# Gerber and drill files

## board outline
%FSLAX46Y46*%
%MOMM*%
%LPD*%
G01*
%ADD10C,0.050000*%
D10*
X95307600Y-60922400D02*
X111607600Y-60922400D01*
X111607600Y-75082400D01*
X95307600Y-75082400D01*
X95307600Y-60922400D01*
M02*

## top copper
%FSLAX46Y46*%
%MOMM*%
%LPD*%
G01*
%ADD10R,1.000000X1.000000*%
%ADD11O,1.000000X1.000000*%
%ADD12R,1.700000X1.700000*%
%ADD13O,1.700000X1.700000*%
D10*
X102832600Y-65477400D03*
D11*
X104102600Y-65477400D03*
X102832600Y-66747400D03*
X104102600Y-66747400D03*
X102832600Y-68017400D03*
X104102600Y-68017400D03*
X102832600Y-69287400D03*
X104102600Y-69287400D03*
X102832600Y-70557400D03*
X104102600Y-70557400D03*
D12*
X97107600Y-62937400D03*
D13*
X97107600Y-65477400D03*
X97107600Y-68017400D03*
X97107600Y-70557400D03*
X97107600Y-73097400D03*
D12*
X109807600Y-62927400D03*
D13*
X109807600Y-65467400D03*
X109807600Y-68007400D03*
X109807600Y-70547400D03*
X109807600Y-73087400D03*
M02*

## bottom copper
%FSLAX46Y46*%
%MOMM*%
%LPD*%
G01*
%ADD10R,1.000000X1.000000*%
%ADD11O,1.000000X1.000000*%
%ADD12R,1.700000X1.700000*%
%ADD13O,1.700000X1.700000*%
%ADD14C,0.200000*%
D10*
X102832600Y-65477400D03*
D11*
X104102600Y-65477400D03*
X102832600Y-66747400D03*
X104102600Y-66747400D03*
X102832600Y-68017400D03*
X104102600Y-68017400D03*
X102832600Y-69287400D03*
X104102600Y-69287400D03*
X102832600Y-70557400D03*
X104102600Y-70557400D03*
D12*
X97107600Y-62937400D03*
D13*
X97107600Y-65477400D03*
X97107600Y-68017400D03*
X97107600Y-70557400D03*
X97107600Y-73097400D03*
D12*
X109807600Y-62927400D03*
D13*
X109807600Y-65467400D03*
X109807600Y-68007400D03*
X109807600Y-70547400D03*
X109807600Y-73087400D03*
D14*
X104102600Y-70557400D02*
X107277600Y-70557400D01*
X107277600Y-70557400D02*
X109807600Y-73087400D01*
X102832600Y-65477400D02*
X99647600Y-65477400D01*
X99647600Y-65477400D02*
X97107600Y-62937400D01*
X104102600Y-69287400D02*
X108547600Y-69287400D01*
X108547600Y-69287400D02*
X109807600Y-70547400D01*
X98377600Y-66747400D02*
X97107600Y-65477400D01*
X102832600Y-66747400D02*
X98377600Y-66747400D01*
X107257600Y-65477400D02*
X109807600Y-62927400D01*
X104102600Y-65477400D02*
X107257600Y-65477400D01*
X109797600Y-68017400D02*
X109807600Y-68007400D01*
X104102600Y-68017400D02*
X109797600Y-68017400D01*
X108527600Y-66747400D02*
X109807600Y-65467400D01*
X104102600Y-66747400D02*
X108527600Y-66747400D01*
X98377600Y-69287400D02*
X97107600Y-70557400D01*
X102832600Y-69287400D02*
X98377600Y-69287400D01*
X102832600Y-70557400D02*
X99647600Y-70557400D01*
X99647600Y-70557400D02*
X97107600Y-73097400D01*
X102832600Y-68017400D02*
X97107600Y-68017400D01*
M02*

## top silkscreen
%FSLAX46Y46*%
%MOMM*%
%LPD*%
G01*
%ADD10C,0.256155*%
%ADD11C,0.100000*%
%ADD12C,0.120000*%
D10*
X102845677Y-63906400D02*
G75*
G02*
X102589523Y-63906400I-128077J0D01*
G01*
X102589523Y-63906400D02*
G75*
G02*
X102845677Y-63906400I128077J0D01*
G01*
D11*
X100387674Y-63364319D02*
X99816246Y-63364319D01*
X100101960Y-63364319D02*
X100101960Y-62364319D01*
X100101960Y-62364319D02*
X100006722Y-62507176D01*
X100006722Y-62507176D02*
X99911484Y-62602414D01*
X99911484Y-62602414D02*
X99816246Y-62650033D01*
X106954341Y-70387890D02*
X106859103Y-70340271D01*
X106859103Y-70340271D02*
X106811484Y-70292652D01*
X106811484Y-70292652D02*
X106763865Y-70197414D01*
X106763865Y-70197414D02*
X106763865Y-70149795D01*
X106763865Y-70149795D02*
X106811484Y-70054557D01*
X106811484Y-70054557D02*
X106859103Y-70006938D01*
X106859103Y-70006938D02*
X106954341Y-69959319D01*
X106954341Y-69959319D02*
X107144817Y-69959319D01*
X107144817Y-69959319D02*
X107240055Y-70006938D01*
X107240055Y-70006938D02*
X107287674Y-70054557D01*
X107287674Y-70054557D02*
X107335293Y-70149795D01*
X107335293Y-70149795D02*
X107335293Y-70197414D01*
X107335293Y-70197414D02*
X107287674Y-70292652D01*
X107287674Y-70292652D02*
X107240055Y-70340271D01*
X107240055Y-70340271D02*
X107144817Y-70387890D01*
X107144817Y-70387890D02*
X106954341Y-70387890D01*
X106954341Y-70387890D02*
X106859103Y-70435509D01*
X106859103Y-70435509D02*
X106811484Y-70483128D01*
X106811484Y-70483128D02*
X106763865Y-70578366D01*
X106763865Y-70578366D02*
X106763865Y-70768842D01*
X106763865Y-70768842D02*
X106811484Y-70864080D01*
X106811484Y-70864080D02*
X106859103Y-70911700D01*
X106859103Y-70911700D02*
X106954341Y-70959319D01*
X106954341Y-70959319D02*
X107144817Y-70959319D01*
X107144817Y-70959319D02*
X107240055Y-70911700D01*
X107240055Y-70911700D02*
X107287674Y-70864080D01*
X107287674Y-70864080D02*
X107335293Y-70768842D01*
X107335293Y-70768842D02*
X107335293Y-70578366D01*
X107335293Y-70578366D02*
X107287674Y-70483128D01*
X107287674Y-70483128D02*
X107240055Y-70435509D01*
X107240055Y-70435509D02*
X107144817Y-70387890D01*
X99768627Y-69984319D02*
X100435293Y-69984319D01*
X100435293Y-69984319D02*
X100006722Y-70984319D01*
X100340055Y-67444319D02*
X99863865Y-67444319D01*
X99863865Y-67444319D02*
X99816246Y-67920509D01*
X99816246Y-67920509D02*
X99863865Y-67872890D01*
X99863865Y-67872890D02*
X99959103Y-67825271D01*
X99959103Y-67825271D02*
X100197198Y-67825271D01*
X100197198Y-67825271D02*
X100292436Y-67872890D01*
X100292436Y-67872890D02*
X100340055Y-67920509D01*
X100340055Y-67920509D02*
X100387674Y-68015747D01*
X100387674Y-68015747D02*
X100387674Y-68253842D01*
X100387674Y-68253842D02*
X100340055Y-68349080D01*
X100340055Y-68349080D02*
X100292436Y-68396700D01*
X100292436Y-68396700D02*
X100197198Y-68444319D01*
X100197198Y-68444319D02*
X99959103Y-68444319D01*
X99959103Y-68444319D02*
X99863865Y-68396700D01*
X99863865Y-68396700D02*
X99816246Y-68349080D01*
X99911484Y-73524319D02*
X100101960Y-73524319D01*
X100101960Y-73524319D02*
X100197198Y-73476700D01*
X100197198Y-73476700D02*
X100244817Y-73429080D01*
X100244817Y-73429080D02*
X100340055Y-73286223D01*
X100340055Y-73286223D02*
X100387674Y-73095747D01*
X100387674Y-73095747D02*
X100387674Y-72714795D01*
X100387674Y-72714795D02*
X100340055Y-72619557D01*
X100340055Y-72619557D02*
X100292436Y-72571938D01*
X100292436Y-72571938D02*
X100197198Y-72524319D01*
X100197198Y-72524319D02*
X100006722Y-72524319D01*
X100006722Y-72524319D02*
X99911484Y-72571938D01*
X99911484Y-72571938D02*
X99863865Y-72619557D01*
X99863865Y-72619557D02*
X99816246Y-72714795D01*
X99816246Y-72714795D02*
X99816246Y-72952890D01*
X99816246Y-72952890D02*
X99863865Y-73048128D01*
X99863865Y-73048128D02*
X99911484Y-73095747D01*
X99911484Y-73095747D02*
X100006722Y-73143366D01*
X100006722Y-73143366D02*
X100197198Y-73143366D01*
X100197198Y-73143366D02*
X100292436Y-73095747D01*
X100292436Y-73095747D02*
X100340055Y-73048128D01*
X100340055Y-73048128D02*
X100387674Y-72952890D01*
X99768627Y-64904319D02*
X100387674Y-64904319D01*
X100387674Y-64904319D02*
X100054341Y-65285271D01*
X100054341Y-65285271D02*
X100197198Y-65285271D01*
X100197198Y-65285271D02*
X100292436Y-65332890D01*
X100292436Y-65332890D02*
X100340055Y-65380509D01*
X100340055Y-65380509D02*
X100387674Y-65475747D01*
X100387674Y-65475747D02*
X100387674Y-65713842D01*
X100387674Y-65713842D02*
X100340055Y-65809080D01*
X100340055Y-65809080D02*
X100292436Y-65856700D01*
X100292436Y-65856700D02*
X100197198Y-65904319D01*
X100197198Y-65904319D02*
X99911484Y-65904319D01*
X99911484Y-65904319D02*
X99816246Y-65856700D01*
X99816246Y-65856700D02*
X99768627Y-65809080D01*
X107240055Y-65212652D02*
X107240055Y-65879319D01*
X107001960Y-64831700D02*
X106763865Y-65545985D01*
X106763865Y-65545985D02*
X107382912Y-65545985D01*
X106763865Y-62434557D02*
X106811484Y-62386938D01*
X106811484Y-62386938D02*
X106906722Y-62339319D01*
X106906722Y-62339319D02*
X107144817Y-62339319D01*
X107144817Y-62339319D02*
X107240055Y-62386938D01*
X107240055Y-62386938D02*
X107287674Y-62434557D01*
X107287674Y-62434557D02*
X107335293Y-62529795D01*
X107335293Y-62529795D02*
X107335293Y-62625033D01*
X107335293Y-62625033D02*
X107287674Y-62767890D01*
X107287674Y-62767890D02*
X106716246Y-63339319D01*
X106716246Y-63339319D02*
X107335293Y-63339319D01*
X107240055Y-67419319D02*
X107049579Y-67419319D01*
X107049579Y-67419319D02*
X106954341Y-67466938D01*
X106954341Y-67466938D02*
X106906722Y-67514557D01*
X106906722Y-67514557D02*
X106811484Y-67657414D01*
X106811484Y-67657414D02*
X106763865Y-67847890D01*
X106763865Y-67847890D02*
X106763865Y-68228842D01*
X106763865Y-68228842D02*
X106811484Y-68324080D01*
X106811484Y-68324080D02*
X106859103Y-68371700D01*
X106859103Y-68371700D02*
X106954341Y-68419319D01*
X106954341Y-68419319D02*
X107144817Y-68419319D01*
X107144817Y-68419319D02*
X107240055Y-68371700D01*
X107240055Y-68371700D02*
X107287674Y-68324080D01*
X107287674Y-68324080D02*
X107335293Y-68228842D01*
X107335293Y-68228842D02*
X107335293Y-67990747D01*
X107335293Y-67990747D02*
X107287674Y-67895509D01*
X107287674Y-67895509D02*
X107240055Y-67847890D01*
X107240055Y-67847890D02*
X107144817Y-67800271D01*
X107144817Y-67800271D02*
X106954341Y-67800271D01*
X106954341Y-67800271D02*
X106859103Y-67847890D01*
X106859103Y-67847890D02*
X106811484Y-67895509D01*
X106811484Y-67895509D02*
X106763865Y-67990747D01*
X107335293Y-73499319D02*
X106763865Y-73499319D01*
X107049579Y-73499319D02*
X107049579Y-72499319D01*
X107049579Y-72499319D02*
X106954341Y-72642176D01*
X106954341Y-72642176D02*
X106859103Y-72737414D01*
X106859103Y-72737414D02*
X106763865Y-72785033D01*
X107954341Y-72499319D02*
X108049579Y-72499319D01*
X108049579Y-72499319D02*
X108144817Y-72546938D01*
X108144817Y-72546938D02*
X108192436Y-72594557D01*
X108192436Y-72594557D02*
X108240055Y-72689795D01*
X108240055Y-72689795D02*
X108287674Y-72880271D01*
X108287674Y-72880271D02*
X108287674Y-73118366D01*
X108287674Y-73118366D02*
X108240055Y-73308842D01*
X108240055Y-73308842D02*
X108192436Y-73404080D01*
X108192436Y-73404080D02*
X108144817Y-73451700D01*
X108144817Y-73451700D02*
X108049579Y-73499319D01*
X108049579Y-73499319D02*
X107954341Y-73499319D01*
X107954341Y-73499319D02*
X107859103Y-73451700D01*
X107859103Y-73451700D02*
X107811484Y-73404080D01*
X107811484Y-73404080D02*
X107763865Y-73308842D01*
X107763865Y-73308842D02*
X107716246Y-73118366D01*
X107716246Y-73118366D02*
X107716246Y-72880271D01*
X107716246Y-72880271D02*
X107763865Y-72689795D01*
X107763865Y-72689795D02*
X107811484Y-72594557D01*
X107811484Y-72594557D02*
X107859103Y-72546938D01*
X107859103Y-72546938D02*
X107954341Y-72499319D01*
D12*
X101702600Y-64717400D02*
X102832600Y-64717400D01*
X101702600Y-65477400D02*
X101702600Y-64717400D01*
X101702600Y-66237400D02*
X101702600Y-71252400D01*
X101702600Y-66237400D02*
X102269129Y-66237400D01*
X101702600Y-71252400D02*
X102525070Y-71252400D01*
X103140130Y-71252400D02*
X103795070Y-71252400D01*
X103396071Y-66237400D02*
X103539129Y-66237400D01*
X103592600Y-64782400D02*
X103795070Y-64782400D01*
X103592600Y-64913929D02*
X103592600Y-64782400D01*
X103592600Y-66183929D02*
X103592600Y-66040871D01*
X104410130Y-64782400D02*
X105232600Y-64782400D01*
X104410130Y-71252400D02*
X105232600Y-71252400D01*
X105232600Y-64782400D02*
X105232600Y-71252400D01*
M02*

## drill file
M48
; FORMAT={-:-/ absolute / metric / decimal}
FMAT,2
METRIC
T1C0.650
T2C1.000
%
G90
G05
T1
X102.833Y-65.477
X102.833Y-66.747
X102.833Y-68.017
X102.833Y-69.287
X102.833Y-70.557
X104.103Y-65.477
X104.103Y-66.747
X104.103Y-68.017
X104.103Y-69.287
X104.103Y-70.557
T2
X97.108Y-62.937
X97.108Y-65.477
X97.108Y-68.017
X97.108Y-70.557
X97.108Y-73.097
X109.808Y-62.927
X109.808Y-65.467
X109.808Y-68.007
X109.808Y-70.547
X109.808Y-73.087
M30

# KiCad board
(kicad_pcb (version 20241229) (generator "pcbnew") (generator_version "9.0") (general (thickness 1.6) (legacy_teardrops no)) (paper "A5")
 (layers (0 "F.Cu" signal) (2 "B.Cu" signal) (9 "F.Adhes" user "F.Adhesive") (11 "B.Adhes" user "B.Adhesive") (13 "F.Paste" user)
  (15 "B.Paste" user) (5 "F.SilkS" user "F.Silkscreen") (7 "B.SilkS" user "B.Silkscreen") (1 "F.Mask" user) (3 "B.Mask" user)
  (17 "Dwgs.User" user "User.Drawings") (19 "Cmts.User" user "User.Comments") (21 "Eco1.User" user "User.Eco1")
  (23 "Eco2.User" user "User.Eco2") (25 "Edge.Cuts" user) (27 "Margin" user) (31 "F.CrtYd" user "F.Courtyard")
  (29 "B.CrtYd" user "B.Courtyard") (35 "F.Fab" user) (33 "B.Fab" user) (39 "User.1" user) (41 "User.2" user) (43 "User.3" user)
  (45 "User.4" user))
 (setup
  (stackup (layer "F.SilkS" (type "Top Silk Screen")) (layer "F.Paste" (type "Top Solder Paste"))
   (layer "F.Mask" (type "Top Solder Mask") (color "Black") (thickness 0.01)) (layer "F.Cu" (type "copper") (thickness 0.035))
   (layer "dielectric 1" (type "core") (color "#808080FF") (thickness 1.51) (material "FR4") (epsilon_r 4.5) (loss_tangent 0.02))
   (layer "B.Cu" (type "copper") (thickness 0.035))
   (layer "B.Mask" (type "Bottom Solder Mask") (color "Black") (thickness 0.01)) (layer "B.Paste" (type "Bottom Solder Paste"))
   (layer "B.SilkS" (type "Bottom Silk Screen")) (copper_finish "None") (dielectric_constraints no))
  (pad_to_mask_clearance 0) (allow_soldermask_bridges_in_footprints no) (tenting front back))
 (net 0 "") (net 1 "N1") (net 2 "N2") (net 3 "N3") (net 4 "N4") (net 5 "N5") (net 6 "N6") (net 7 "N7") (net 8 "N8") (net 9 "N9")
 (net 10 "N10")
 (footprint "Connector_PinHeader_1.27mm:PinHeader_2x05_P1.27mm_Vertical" (layer "F.Cu") (at 102.8326 65.4774)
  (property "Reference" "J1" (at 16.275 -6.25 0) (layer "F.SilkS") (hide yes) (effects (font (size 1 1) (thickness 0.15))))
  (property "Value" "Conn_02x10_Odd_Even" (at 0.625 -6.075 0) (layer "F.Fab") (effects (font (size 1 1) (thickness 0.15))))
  (fp_line (start -1.13 -0.76) (end 0 -0.76) (stroke (width 0.12) (type solid)) (layer "F.SilkS"))
  (fp_line (start -1.13 0) (end -1.13 -0.76) (stroke (width 0.12) (type solid)) (layer "F.SilkS"))
  (fp_line (start -1.13 0.76) (end -1.13 5.775) (stroke (width 0.12) (type solid)) (layer "F.SilkS"))
  (fp_line (start -1.13 0.76) (end -0.563471 0.76) (stroke (width 0.12) (type solid)) (layer "F.SilkS"))
  (fp_line (start -1.13 5.775) (end -0.30753 5.775) (stroke (width 0.12) (type solid)) (layer "F.SilkS"))
  (fp_line (start 0.30753 5.775) (end 0.96247 5.775) (stroke (width 0.12) (type solid)) (layer "F.SilkS"))
  (fp_line (start 0.563471 0.76) (end 0.706529 0.76) (stroke (width 0.12) (type solid)) (layer "F.SilkS"))
  (fp_line (start 0.76 -0.695) (end 0.96247 -0.695) (stroke (width 0.12) (type solid)) (layer "F.SilkS"))
  (fp_line (start 0.76 -0.563471) (end 0.76 -0.695) (stroke (width 0.12) (type solid)) (layer "F.SilkS"))
  (fp_line (start 0.76 0.706529) (end 0.76 0.563471) (stroke (width 0.12) (type solid)) (layer "F.SilkS"))
  (fp_line (start 1.57753 -0.695) (end 2.4 -0.695) (stroke (width 0.12) (type solid)) (layer "F.SilkS"))
  (fp_line (start 1.57753 5.775) (end 2.4 5.775) (stroke (width 0.12) (type solid)) (layer "F.SilkS"))
  (fp_line (start 2.4 -0.695) (end 2.4 5.775) (stroke (width 0.12) (type solid)) (layer "F.SilkS"))
  (pad "1" thru_hole rect (at 0 0) (size 1 1) (drill 0.65) (layers "*.Cu" "*.Mask") (remove_unused_layers no) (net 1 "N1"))
  (pad "2" thru_hole oval (at 1.27 0) (size 1 1) (drill 0.65) (layers "*.Cu" "*.Mask") (remove_unused_layers no) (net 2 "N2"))
  (pad "3" thru_hole oval (at 0 1.27) (size 1 1) (drill 0.65) (layers "*.Cu" "*.Mask") (remove_unused_layers no) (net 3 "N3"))
  (pad "4" thru_hole oval (at 1.27 1.27) (size 1 1) (drill 0.65) (layers "*.Cu" "*.Mask") (remove_unused_layers no) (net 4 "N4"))
  (pad "5" thru_hole oval (at 0 2.54) (size 1 1) (drill 0.65) (layers "*.Cu" "*.Mask") (remove_unused_layers no) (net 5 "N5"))
  (pad "6" thru_hole oval (at 1.27 2.54) (size 1 1) (drill 0.65) (layers "*.Cu" "*.Mask") (remove_unused_layers no) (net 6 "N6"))
  (pad "7" thru_hole oval (at 0 3.81) (size 1 1) (drill 0.65) (layers "*.Cu" "*.Mask") (remove_unused_layers no) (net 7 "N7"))
  (pad "8" thru_hole oval (at 1.27 3.81) (size 1 1) (drill 0.65) (layers "*.Cu" "*.Mask") (remove_unused_layers no) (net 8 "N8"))
  (pad "9" thru_hole oval (at 0 5.08) (size 1 1) (drill 0.65) (layers "*.Cu" "*.Mask") (remove_unused_layers no) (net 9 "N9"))
  (pad "10" thru_hole oval (at 1.27 5.08) (size 1 1) (drill 0.65) (layers "*.Cu" "*.Mask") (remove_unused_layers no) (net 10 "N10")))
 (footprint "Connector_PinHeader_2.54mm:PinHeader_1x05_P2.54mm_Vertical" (layer "B.Cu") (at 97.1076 62.9374 180)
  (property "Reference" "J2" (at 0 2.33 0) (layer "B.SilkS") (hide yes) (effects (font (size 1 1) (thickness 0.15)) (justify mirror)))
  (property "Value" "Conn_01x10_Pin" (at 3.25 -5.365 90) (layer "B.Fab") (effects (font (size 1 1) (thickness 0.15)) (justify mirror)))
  (pad "1" thru_hole rect (at 0 0 180) (size 1.7 1.7) (drill 1) (layers "*.Cu" "*.Mask") (remove_unused_layers no) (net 1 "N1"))
  (pad "2" thru_hole oval (at 0 -2.54 180) (size 1.7 1.7) (drill 1) (layers "*.Cu" "*.Mask") (remove_unused_layers no) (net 3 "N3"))
  (pad "3" thru_hole oval (at 0 -5.08 180) (size 1.7 1.7) (drill 1) (layers "*.Cu" "*.Mask") (remove_unused_layers no) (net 5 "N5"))
  (pad "4" thru_hole oval (at 0 -7.62 180) (size 1.7 1.7) (drill 1) (layers "*.Cu" "*.Mask") (remove_unused_layers no) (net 7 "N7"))
  (pad "5" thru_hole oval (at 0 -10.16 180) (size 1.7 1.7) (drill 1) (layers "*.Cu" "*.Mask") (remove_unused_layers no) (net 9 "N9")))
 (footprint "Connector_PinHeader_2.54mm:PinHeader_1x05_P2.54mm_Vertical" (layer "B.Cu") (at 109.8076 62.9274 180)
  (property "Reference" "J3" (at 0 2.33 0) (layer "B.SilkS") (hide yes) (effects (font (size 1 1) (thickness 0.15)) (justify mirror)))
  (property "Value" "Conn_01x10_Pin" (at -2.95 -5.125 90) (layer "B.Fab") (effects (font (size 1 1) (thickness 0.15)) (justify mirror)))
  (pad "1" thru_hole rect (at 0 0 180) (size 1.7 1.7) (drill 1) (layers "*.Cu" "*.Mask") (remove_unused_layers no) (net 2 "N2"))
  (pad "2" thru_hole oval (at 0 -2.54 180) (size 1.7 1.7) (drill 1) (layers "*.Cu" "*.Mask") (remove_unused_layers no) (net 4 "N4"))
  (pad "3" thru_hole oval (at 0 -5.08 180) (size 1.7 1.7) (drill 1) (layers "*.Cu" "*.Mask") (remove_unused_layers no) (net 6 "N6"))
  (pad "4" thru_hole oval (at 0 -7.62 180) (size 1.7 1.7) (drill 1) (layers "*.Cu" "*.Mask") (remove_unused_layers no) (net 8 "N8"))
  (pad "5" thru_hole oval (at 0 -10.16 180) (size 1.7 1.7) (drill 1) (layers "*.Cu" "*.Mask") (remove_unused_layers no) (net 10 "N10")))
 (gr_circle (center 102.7176 63.9064) (end 102.5176 63.9564) (stroke (width 0.1) (type solid)) (fill yes) (layer "F.SilkS"))
 (gr_rect (start 95.3076 60.9224) (end 111.6076 75.0824) (stroke (width 0.05) (type default)) (fill no) (layer "Edge.Cuts"))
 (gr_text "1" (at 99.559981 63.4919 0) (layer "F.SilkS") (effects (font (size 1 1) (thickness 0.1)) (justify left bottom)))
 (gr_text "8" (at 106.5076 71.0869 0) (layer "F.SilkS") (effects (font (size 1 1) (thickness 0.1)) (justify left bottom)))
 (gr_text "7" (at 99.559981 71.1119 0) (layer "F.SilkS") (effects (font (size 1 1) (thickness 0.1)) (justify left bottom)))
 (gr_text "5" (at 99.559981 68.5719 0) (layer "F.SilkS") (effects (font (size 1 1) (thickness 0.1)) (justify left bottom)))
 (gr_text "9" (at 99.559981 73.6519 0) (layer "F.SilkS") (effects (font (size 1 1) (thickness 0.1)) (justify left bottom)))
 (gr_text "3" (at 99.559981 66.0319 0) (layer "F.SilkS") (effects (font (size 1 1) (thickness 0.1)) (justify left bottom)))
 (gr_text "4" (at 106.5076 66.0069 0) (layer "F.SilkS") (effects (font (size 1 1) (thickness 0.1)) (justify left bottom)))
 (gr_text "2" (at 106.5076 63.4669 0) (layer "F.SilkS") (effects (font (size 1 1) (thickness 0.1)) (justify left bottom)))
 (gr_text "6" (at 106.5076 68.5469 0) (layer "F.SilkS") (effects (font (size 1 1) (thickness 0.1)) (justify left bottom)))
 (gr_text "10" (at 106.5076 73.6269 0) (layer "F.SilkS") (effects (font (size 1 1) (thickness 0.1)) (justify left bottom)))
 (segment (start 104.1026 70.5574) (end 107.2776 70.5574) (width 0.2) (layer "B.Cu") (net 10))
 (segment (start 107.2776 70.5574) (end 109.8076 73.0874) (width 0.2) (layer "B.Cu") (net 10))
 (segment (start 102.8326 65.4774) (end 99.6476 65.4774) (width 0.2) (layer "B.Cu") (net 1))
 (segment (start 99.6476 65.4774) (end 97.1076 62.9374) (width 0.2) (layer "B.Cu") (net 1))
 (segment (start 104.1026 69.2874) (end 108.5476 69.2874) (width 0.2) (layer "B.Cu") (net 8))
 (segment (start 108.5476 69.2874) (end 109.8076 70.5474) (width 0.2) (layer "B.Cu") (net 8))
 (segment (start 98.3776 66.7474) (end 97.1076 65.4774) (width 0.2) (layer "B.Cu") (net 3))
 (segment (start 102.8326 66.7474) (end 98.3776 66.7474) (width 0.2) (layer "B.Cu") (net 3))
 (segment (start 107.2576 65.4774) (end 109.8076 62.9274) (width 0.2) (layer "B.Cu") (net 2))
 (segment (start 104.1026 65.4774) (end 107.2576 65.4774) (width 0.2) (layer "B.Cu") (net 2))
 (segment (start 109.7976 68.0174) (end 109.8076 68.0074) (width 0.2) (layer "B.Cu") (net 6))
 (segment (start 104.1026 68.0174) (end 109.7976 68.0174) (width 0.2) (layer "B.Cu") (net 6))
 (segment (start 108.5276 66.7474) (end 109.8076 65.4674) (width 0.2) (layer "B.Cu") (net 4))
 (segment (start 104.1026 66.7474) (end 108.5276 66.7474) (width 0.2) (layer "B.Cu") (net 4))
 (segment (start 98.3776 69.2874) (end 97.1076 70.5574) (width 0.2) (layer "B.Cu") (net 7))
 (segment (start 102.8326 69.2874) (end 98.3776 69.2874) (width 0.2) (layer "B.Cu") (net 7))
 (segment (start 102.8326 70.5574) (end 99.6476 70.5574) (width 0.2) (layer "B.Cu") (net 9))
 (segment (start 99.6476 70.5574) (end 97.1076 73.0974) (width 0.2) (layer "B.Cu") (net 9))
 (segment (start 102.8326 68.0174) (end 97.1076 68.0174) (width 0.2) (layer "B.Cu") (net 5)))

